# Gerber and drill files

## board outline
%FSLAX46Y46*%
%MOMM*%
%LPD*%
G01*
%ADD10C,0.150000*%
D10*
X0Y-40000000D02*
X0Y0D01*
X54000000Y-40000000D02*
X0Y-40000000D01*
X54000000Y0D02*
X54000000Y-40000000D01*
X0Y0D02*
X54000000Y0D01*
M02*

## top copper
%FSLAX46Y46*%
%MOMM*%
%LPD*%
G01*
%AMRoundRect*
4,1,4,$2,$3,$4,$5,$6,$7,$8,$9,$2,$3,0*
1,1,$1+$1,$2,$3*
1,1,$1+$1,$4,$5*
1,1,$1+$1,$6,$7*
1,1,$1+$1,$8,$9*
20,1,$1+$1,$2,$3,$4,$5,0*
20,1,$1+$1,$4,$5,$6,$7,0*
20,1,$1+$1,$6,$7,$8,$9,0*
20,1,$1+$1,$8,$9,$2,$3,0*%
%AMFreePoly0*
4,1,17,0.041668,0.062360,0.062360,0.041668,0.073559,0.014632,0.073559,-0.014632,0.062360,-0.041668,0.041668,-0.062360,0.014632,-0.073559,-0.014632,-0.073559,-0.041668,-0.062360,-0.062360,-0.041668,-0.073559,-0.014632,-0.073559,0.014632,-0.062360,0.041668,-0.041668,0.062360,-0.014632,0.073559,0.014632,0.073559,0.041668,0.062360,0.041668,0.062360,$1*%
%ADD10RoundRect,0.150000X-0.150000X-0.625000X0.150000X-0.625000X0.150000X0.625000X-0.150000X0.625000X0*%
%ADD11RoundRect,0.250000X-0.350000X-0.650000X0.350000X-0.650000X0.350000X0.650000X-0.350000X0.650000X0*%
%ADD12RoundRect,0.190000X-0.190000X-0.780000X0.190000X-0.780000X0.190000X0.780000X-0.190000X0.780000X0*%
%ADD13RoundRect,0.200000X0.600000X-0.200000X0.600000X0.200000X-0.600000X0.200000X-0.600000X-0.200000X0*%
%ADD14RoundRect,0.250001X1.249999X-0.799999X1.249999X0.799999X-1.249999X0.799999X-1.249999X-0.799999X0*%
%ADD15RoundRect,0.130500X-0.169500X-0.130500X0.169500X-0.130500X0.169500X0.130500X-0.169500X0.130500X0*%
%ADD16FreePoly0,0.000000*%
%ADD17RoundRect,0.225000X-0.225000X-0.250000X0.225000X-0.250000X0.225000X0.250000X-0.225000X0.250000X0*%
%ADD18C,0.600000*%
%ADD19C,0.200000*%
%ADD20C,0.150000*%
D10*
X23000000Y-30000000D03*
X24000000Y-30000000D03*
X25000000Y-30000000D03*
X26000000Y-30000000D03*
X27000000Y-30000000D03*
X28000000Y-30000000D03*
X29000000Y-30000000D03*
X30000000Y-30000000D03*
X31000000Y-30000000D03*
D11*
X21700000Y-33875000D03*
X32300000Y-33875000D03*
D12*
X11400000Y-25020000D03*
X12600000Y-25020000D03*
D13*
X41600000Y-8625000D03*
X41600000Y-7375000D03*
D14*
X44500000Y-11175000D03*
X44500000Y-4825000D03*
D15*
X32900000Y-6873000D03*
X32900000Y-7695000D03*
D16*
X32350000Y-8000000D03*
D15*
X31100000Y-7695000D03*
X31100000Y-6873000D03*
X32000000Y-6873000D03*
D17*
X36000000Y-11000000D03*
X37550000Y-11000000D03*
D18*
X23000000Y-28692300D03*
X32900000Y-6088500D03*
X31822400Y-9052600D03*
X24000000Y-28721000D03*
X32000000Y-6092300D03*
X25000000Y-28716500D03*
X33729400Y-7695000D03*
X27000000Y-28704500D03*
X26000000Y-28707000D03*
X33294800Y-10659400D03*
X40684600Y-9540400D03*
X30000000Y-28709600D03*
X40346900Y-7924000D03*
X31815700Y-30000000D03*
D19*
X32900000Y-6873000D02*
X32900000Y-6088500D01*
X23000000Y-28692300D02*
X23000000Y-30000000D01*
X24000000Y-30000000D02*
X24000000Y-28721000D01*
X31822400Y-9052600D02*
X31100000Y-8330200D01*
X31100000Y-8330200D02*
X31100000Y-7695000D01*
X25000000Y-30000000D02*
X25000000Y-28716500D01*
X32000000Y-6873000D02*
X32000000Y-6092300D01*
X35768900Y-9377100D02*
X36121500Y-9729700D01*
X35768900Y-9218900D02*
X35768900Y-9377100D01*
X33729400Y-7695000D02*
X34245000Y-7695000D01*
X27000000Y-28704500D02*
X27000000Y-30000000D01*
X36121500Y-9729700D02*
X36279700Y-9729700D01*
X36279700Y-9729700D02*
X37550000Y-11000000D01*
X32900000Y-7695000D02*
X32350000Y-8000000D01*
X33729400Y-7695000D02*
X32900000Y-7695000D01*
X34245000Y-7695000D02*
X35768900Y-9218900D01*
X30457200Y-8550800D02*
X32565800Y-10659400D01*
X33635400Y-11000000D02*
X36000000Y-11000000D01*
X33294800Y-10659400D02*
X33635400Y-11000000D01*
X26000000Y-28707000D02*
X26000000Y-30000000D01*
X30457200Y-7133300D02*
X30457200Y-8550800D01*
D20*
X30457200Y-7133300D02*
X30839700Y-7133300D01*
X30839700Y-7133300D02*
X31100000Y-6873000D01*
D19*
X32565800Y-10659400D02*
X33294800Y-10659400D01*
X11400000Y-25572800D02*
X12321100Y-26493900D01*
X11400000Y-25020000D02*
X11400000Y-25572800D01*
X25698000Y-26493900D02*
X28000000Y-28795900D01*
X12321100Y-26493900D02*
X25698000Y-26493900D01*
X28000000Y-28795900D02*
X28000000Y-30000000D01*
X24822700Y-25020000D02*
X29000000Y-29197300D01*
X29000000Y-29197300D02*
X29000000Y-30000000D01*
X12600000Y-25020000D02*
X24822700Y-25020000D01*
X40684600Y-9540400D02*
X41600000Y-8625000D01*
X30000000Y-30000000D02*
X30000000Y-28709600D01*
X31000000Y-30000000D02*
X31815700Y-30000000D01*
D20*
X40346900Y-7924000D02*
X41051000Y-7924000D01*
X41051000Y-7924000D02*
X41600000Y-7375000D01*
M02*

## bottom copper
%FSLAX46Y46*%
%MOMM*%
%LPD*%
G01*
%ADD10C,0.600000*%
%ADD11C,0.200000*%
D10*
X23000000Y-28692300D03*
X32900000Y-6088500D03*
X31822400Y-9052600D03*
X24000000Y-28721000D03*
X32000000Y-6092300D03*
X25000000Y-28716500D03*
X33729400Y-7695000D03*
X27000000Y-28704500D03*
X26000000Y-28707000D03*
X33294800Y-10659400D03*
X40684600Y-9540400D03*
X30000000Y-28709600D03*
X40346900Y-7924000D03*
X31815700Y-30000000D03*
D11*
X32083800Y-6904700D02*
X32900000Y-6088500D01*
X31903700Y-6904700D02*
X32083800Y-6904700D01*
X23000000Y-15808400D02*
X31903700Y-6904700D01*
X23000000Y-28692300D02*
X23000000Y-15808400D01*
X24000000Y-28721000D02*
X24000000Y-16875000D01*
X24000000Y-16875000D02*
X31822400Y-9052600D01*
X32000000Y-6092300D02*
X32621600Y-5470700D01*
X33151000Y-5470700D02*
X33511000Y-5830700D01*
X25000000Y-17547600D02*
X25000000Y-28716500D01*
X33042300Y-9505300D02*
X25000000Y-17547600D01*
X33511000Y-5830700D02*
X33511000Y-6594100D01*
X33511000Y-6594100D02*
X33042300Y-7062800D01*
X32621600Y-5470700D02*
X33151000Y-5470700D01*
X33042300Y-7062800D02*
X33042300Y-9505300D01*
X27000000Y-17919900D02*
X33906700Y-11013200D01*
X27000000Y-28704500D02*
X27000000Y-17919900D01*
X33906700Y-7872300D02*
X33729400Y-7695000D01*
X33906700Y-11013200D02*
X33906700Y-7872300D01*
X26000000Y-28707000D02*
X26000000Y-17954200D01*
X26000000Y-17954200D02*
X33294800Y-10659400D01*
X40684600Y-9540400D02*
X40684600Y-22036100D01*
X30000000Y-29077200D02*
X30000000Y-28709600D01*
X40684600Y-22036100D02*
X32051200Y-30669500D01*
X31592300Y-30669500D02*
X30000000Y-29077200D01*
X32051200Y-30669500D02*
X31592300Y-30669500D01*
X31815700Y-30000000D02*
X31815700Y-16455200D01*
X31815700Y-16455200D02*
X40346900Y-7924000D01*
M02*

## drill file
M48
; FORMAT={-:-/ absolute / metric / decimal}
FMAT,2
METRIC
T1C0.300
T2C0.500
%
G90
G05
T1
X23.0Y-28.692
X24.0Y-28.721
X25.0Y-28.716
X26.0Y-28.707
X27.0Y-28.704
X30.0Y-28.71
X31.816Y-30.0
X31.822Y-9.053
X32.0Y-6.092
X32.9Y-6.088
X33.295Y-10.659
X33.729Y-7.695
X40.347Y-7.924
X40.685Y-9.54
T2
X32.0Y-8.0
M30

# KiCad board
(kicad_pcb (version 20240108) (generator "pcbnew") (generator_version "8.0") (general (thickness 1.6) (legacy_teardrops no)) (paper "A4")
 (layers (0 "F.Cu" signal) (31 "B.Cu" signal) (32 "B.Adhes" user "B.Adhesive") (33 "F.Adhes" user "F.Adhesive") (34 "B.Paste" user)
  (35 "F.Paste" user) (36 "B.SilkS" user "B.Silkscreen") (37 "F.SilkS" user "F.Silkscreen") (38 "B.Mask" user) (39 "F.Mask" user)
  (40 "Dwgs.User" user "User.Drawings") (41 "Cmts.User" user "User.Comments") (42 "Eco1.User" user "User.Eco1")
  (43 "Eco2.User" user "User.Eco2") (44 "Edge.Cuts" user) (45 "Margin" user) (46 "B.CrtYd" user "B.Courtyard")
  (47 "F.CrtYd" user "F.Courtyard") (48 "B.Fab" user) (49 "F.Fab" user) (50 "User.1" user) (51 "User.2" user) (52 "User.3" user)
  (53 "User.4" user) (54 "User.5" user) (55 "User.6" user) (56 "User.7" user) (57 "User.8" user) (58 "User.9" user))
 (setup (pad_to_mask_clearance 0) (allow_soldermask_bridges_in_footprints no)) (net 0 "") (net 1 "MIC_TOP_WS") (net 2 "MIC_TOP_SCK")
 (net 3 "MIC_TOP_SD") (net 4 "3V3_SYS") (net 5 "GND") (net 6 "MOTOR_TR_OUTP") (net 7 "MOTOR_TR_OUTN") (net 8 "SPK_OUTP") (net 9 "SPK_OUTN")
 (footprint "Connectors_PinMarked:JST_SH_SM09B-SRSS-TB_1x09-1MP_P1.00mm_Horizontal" (layer "F.Cu") (at 27 32)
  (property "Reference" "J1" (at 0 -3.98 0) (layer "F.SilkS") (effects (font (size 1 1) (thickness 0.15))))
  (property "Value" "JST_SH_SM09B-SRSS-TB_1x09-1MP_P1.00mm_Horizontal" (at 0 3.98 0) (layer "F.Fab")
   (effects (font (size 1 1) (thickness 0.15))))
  (pad "1" smd roundrect (at -4 -2) (size 0.6 1.55) (layers "F.Cu" "F.Paste" "F.Mask") (roundrect_rratio 0.25) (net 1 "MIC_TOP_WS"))
  (pad "2" smd roundrect (at -3 -2) (size 0.6 1.55) (layers "F.Cu" "F.Paste" "F.Mask") (roundrect_rratio 0.25) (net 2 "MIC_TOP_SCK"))
  (pad "3" smd roundrect (at -2 -2) (size 0.6 1.55) (layers "F.Cu" "F.Paste" "F.Mask") (roundrect_rratio 0.25) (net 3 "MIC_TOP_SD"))
  (pad "4" smd roundrect (at -1 -2) (size 0.6 1.55) (layers "F.Cu" "F.Paste" "F.Mask") (roundrect_rratio 0.25) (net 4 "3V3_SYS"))
  (pad "5" smd roundrect (at 0 -2) (size 0.6 1.55) (layers "F.Cu" "F.Paste" "F.Mask") (roundrect_rratio 0.25) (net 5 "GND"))
  (pad "6" smd roundrect (at 1 -2) (size 0.6 1.55) (layers "F.Cu" "F.Paste" "F.Mask") (roundrect_rratio 0.25) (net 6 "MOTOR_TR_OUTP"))
  (pad "7" smd roundrect (at 2 -2) (size 0.6 1.55) (layers "F.Cu" "F.Paste" "F.Mask") (roundrect_rratio 0.25) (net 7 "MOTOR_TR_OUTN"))
  (pad "8" smd roundrect (at 3 -2) (size 0.6 1.55) (layers "F.Cu" "F.Paste" "F.Mask") (roundrect_rratio 0.25) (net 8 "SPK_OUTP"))
  (pad "9" smd roundrect (at 4 -2) (size 0.6 1.55) (layers "F.Cu" "F.Paste" "F.Mask") (roundrect_rratio 0.25) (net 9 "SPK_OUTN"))
  (pad "MP" smd roundrect (at -5.3 1.875) (size 1.2 1.8) (layers "F.Cu" "F.Paste" "F.Mask") (roundrect_rratio 0.208333))
  (pad "MP" smd roundrect (at 5.3 1.875) (size 1.2 1.8) (layers "F.Cu" "F.Paste" "F.Mask") (roundrect_rratio 0.208333)))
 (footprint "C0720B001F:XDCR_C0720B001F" (layer "F.Cu") (at 12 20)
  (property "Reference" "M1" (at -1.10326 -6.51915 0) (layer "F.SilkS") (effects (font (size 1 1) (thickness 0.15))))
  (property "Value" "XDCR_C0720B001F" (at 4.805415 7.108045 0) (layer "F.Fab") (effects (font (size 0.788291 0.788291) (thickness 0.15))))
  (pad "1" smd roundrect (at -0.6 5.02) (size 0.76 1.94) (layers "F.Cu" "F.Paste" "F.Mask") (roundrect_rratio 0.25) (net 6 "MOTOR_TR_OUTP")
   (solder_mask_margin 0.102))
  (pad "2" smd roundrect (at 0.6 5.02) (size 0.76 1.94) (layers "F.Cu" "F.Paste" "F.Mask") (roundrect_rratio 0.25) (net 7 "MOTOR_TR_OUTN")
   (solder_mask_margin 0.102)))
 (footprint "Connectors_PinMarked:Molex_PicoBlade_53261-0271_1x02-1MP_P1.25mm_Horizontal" (layer "F.Cu") (at 44 8 90)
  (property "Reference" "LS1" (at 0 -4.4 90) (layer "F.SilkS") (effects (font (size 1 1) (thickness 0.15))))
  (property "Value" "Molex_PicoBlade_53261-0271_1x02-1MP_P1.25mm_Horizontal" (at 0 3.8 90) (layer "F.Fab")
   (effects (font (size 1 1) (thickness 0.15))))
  (pad "1" smd roundrect (at -0.625 -2.4 90) (size 0.8 1.6) (layers "F.Cu" "F.Paste" "F.Mask") (roundrect_rratio 0.25) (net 8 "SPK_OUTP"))
  (pad "2" smd roundrect (at 0.625 -2.4 90) (size 0.8 1.6) (layers "F.Cu" "F.Paste" "F.Mask") (roundrect_rratio 0.25) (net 9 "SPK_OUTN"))
  (pad "MP" smd roundrect (at -3.175 0.5 90) (size 2.1 3) (layers "F.Cu" "F.Paste" "F.Mask") (roundrect_rratio 0.119048))
  (pad "MP" smd roundrect (at 3.175 0.5 90) (size 2.1 3) (layers "F.Cu" "F.Paste" "F.Mask") (roundrect_rratio 0.119048)))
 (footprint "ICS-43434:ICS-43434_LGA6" (layer "F.Cu") (at 32 8)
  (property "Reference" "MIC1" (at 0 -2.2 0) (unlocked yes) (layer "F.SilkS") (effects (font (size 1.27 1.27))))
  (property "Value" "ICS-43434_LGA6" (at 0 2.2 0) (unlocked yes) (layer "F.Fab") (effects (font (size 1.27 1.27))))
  (pad "1" smd roundrect (at 0.9 -1.127) (size 0.6 0.522) (layers "F.Cu" "F.Paste" "F.Mask") (roundrect_rratio 0.25) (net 1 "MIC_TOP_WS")
   (thermal_bridge_angle 45))
  (pad "2" smd roundrect (at 0.9 -0.305) (size 0.6 0.522) (layers "F.Cu" "F.Paste" "F.Mask") (roundrect_rratio 0.25) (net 5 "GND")
   (thermal_bridge_angle 45))
  (pad "3" smd custom (at 0.35 0) (size 0.15 0.15) (layers "F.Cu" "F.Mask") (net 5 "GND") (options (clearance outline) (anchor circle))
   (primitives))
  (pad "4" smd roundrect (at -0.9 -0.305) (size 0.6 0.522) (layers "F.Cu" "F.Paste" "F.Mask") (roundrect_rratio 0.25) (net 2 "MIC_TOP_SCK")
   (thermal_bridge_angle 45))
  (pad "5" smd roundrect (at -0.9 -1.127) (size 0.6 0.522) (layers "F.Cu" "F.Paste" "F.Mask") (roundrect_rratio 0.25) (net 4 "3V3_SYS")
   (thermal_bridge_angle 45))
  (pad "6" smd roundrect (at 0 -1.127) (size 0.6 0.522) (layers "F.Cu" "F.Paste" "F.Mask") (roundrect_rratio 0.25) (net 3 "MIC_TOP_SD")
   (thermal_bridge_angle 45)))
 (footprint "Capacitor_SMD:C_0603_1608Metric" (layer "F.Cu") (at 36.775 11)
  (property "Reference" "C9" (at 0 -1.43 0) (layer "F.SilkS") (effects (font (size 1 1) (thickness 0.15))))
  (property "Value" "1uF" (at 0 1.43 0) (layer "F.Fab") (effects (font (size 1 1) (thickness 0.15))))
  (pad "1" smd roundrect (at -0.775 0) (size 0.9 0.95) (layers "F.Cu" "F.Paste" "F.Mask") (roundrect_rratio 0.25) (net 4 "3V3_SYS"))
  (pad "2" smd roundrect (at 0.775 0) (size 0.9 0.95) (layers "F.Cu" "F.Paste" "F.Mask") (roundrect_rratio 0.25) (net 5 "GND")))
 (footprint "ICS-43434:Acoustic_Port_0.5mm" (layer "F.Cu") (at 32 8)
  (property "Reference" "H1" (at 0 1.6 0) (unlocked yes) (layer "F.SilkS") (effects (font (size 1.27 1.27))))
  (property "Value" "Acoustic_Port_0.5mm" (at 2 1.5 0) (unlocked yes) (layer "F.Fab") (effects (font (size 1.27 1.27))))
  (pad "" np_thru_hole circle (at 0 0) (size 0.5 0.5) (drill 0.5) (layers "*.Cu" "*.Mask")))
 (gr_line (start 0 40) (end 0 0) (stroke (width 0.15) (type default)) (layer "Edge.Cuts"))
 (gr_line (start 54 40) (end 0 40) (stroke (width 0.15) (type default)) (layer "Edge.Cuts"))
 (gr_line (start 54 0) (end 54 40) (stroke (width 0.15) (type default)) (layer "Edge.Cuts"))
 (gr_line (start 0 0) (end 54 0) (stroke (width 0.15) (type default)) (layer "Edge.Cuts"))
 (segment (start 32.9 6.873) (end 32.9 6.0885) (width 0.2) (layer "F.Cu") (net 1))
 (segment (start 23 28.6923) (end 23 30) (width 0.2) (layer "F.Cu") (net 1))
 (via (at 23 28.6923) (size 0.6) (drill 0.3) (layers "F.Cu" "B.Cu") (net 1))
 (via (at 32.9 6.0885) (size 0.6) (drill 0.3) (layers "F.Cu" "B.Cu") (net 1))
 (segment (start 32.0838 6.9047) (end 32.9 6.0885) (width 0.2) (layer "B.Cu") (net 1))
 (segment (start 31.9037 6.9047) (end 32.0838 6.9047) (width 0.2) (layer "B.Cu") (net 1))
 (segment (start 23 15.8084) (end 31.9037 6.9047) (width 0.2) (layer "B.Cu") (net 1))
 (segment (start 23 28.6923) (end 23 15.8084) (width 0.2) (layer "B.Cu") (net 1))
 (segment (start 24 30) (end 24 28.721) (width 0.2) (layer "F.Cu") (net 2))
 (segment (start 31.8224 9.0526) (end 31.1 8.3302) (width 0.2) (layer "F.Cu") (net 2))
 (segment (start 31.1 8.3302) (end 31.1 7.695) (width 0.2) (layer "F.Cu") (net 2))
 (via (at 31.8224 9.0526) (size 0.6) (drill 0.3) (layers "F.Cu" "B.Cu") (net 2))
 (via (at 24 28.721) (size 0.6) (drill 0.3) (layers "F.Cu" "B.Cu") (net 2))
 (segment (start 24 28.721) (end 24 16.875) (width 0.2) (layer "B.Cu") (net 2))
 (segment (start 24 16.875) (end 31.8224 9.0526) (width 0.2) (layer "B.Cu") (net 2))
 (segment (start 25 30) (end 25 28.7165) (width 0.2) (layer "F.Cu") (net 3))
 (segment (start 32 6.873) (end 32 6.0923) (width 0.2) (layer "F.Cu") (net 3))
 (via (at 32 6.0923) (size 0.6) (drill 0.3) (layers "F.Cu" "B.Cu") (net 3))
 (via (at 25 28.7165) (size 0.6) (drill 0.3) (layers "F.Cu" "B.Cu") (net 3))
 (segment (start 32 6.0923) (end 32.6216 5.4707) (width 0.2) (layer "B.Cu") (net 3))
 (segment (start 33.151 5.4707) (end 33.511 5.8307) (width 0.2) (layer "B.Cu") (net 3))
 (segment (start 25 17.5476) (end 25 28.7165) (width 0.2) (layer "B.Cu") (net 3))
 (segment (start 33.0423 9.5053) (end 25 17.5476) (width 0.2) (layer "B.Cu") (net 3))
 (segment (start 33.511 5.8307) (end 33.511 6.5941) (width 0.2) (layer "B.Cu") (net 3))
 (segment (start 33.511 6.5941) (end 33.0423 7.0628) (width 0.2) (layer "B.Cu") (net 3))
 (segment (start 32.6216 5.4707) (end 33.151 5.4707) (width 0.2) (layer "B.Cu") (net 3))
 (segment (start 33.0423 7.0628) (end 33.0423 9.5053) (width 0.2) (layer "B.Cu") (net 3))
 (segment (start 35.7689 9.3771) (end 36.1215 9.7297) (width 0.2) (layer "F.Cu") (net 5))
 (segment (start 35.7689 9.2189) (end 35.7689 9.3771) (width 0.2) (layer "F.Cu") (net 5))
 (segment (start 33.7294 7.695) (end 34.245 7.695) (width 0.2) (layer "F.Cu") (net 5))
 (segment (start 27 28.7045) (end 27 30) (width 0.2) (layer "F.Cu") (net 5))
 (segment (start 36.1215 9.7297) (end 36.2797 9.7297) (width 0.2) (layer "F.Cu") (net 5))
 (segment (start 36.2797 9.7297) (end 37.55 11) (width 0.2) (layer "F.Cu") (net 5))
 (segment (start 32.9 7.695) (end 32.35 8) (width 0.2) (layer "F.Cu") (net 5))
 (segment (start 33.7294 7.695) (end 32.9 7.695) (width 0.2) (layer "F.Cu") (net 5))
 (segment (start 34.245 7.695) (end 35.7689 9.2189) (width 0.2) (layer "F.Cu") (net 5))
 (via (at 33.7294 7.695) (size 0.6) (drill 0.3) (layers "F.Cu" "B.Cu") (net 5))
 (via (at 27 28.7045) (size 0.6) (drill 0.3) (layers "F.Cu" "B.Cu") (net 5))
 (segment (start 27 17.9199) (end 33.9067 11.0132) (width 0.2) (layer "B.Cu") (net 5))
 (segment (start 27 28.7045) (end 27 17.9199) (width 0.2) (layer "B.Cu") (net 5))
 (segment (start 33.9067 7.8723) (end 33.7294 7.695) (width 0.2) (layer "B.Cu") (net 5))
 (segment (start 33.9067 11.0132) (end 33.9067 7.8723) (width 0.2) (layer "B.Cu") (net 5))
 (segment (start 30.4572 8.5508) (end 32.5658 10.6594) (width 0.2) (layer "F.Cu") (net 4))
 (segment (start 33.6354 11) (end 36 11) (width 0.2) (layer "F.Cu") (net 4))
 (segment (start 33.2948 10.6594) (end 33.6354 11) (width 0.2) (layer "F.Cu") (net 4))
 (segment (start 26 28.707) (end 26 30) (width 0.2) (layer "F.Cu") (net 4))
 (segment (start 30.4572 7.1333) (end 30.4572 8.5508) (width 0.2) (layer "F.Cu") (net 4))
 (segment (start 30.4572 7.1333) (end 30.8397 7.1333) (width 0.15) (layer "F.Cu") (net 4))
 (segment (start 30.8397 7.1333) (end 31.1 6.873) (width 0.15) (layer "F.Cu") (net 4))
 (segment (start 32.5658 10.6594) (end 33.2948 10.6594) (width 0.2) (layer "F.Cu") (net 4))
 (via (at 26 28.707) (size 0.6) (drill 0.3) (layers "F.Cu" "B.Cu") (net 4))
 (via (at 33.2948 10.6594) (size 0.6) (drill 0.3) (layers "F.Cu" "B.Cu") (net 4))
 (segment (start 26 28.707) (end 26 17.9542) (width 0.2) (layer "B.Cu") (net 4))
 (segment (start 26 17.9542) (end 33.2948 10.6594) (width 0.2) (layer "B.Cu") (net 4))
 (segment (start 11.4 25.5728) (end 12.3211 26.4939) (width 0.2) (layer "F.Cu") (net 6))
 (segment (start 11.4 25.02) (end 11.4 25.5728) (width 0.2) (layer "F.Cu") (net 6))
 (segment (start 25.698 26.4939) (end 28 28.7959) (width 0.2) (layer "F.Cu") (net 6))
 (segment (start 12.3211 26.4939) (end 25.698 26.4939) (width 0.2) (layer "F.Cu") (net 6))
 (segment (start 28 28.7959) (end 28 30) (width 0.2) (layer "F.Cu") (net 6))
 (segment (start 24.8227 25.02) (end 29 29.1973) (width 0.2) (layer "F.Cu") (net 7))
 (segment (start 29 29.1973) (end 29 30) (width 0.2) (layer "F.Cu") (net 7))
 (segment (start 12.6 25.02) (end 24.8227 25.02) (width 0.2) (layer "F.Cu") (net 7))
 (segment (start 40.6846 9.5404) (end 41.6 8.625) (width 0.2) (layer "F.Cu") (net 8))
 (segment (start 30 30) (end 30 28.7096) (width 0.2) (layer "F.Cu") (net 8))
 (via (at 40.6846 9.5404) (size 0.6) (drill 0.3) (layers "F.Cu" "B.Cu") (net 8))
 (via (at 30 28.7096) (size 0.6) (drill 0.3) (layers "F.Cu" "B.Cu") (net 8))
 (segment (start 40.6846 9.5404) (end 40.6846 22.0361) (width 0.2) (layer "B.Cu") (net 8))
 (segment (start 30 29.0772) (end 30 28.7096) (width 0.2) (layer "B.Cu") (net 8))
 (segment (start 40.6846 22.0361) (end 32.0512 30.6695) (width 0.2) (layer "B.Cu") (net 8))
 (segment (start 31.5923 30.6695) (end 30 29.0772) (width 0.2) (layer "B.Cu") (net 8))
 (segment (start 32.0512 30.6695) (end 31.5923 30.6695) (width 0.2) (layer "B.Cu") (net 8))
 (segment (start 31 30) (end 31.8157 30) (width 0.2) (layer "F.Cu") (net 9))
 (segment (start 40.3469 7.924) (end 41.051 7.924) (width 0.15) (layer "F.Cu") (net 9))
 (segment (start 41.051 7.924) (end 41.6 7.375) (width 0.15) (layer "F.Cu") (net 9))
 (via (at 40.3469 7.924) (size 0.6) (drill 0.3) (layers "F.Cu" "B.Cu") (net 9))
 (via (at 31.8157 30) (size 0.6) (drill 0.3) (layers "F.Cu" "B.Cu") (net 9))
 (segment (start 31.8157 30) (end 31.8157 16.4552) (width 0.2) (layer "B.Cu") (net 9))
 (segment (start 31.8157 16.4552) (end 40.3469 7.924) (width 0.2) (layer "B.Cu") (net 9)))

